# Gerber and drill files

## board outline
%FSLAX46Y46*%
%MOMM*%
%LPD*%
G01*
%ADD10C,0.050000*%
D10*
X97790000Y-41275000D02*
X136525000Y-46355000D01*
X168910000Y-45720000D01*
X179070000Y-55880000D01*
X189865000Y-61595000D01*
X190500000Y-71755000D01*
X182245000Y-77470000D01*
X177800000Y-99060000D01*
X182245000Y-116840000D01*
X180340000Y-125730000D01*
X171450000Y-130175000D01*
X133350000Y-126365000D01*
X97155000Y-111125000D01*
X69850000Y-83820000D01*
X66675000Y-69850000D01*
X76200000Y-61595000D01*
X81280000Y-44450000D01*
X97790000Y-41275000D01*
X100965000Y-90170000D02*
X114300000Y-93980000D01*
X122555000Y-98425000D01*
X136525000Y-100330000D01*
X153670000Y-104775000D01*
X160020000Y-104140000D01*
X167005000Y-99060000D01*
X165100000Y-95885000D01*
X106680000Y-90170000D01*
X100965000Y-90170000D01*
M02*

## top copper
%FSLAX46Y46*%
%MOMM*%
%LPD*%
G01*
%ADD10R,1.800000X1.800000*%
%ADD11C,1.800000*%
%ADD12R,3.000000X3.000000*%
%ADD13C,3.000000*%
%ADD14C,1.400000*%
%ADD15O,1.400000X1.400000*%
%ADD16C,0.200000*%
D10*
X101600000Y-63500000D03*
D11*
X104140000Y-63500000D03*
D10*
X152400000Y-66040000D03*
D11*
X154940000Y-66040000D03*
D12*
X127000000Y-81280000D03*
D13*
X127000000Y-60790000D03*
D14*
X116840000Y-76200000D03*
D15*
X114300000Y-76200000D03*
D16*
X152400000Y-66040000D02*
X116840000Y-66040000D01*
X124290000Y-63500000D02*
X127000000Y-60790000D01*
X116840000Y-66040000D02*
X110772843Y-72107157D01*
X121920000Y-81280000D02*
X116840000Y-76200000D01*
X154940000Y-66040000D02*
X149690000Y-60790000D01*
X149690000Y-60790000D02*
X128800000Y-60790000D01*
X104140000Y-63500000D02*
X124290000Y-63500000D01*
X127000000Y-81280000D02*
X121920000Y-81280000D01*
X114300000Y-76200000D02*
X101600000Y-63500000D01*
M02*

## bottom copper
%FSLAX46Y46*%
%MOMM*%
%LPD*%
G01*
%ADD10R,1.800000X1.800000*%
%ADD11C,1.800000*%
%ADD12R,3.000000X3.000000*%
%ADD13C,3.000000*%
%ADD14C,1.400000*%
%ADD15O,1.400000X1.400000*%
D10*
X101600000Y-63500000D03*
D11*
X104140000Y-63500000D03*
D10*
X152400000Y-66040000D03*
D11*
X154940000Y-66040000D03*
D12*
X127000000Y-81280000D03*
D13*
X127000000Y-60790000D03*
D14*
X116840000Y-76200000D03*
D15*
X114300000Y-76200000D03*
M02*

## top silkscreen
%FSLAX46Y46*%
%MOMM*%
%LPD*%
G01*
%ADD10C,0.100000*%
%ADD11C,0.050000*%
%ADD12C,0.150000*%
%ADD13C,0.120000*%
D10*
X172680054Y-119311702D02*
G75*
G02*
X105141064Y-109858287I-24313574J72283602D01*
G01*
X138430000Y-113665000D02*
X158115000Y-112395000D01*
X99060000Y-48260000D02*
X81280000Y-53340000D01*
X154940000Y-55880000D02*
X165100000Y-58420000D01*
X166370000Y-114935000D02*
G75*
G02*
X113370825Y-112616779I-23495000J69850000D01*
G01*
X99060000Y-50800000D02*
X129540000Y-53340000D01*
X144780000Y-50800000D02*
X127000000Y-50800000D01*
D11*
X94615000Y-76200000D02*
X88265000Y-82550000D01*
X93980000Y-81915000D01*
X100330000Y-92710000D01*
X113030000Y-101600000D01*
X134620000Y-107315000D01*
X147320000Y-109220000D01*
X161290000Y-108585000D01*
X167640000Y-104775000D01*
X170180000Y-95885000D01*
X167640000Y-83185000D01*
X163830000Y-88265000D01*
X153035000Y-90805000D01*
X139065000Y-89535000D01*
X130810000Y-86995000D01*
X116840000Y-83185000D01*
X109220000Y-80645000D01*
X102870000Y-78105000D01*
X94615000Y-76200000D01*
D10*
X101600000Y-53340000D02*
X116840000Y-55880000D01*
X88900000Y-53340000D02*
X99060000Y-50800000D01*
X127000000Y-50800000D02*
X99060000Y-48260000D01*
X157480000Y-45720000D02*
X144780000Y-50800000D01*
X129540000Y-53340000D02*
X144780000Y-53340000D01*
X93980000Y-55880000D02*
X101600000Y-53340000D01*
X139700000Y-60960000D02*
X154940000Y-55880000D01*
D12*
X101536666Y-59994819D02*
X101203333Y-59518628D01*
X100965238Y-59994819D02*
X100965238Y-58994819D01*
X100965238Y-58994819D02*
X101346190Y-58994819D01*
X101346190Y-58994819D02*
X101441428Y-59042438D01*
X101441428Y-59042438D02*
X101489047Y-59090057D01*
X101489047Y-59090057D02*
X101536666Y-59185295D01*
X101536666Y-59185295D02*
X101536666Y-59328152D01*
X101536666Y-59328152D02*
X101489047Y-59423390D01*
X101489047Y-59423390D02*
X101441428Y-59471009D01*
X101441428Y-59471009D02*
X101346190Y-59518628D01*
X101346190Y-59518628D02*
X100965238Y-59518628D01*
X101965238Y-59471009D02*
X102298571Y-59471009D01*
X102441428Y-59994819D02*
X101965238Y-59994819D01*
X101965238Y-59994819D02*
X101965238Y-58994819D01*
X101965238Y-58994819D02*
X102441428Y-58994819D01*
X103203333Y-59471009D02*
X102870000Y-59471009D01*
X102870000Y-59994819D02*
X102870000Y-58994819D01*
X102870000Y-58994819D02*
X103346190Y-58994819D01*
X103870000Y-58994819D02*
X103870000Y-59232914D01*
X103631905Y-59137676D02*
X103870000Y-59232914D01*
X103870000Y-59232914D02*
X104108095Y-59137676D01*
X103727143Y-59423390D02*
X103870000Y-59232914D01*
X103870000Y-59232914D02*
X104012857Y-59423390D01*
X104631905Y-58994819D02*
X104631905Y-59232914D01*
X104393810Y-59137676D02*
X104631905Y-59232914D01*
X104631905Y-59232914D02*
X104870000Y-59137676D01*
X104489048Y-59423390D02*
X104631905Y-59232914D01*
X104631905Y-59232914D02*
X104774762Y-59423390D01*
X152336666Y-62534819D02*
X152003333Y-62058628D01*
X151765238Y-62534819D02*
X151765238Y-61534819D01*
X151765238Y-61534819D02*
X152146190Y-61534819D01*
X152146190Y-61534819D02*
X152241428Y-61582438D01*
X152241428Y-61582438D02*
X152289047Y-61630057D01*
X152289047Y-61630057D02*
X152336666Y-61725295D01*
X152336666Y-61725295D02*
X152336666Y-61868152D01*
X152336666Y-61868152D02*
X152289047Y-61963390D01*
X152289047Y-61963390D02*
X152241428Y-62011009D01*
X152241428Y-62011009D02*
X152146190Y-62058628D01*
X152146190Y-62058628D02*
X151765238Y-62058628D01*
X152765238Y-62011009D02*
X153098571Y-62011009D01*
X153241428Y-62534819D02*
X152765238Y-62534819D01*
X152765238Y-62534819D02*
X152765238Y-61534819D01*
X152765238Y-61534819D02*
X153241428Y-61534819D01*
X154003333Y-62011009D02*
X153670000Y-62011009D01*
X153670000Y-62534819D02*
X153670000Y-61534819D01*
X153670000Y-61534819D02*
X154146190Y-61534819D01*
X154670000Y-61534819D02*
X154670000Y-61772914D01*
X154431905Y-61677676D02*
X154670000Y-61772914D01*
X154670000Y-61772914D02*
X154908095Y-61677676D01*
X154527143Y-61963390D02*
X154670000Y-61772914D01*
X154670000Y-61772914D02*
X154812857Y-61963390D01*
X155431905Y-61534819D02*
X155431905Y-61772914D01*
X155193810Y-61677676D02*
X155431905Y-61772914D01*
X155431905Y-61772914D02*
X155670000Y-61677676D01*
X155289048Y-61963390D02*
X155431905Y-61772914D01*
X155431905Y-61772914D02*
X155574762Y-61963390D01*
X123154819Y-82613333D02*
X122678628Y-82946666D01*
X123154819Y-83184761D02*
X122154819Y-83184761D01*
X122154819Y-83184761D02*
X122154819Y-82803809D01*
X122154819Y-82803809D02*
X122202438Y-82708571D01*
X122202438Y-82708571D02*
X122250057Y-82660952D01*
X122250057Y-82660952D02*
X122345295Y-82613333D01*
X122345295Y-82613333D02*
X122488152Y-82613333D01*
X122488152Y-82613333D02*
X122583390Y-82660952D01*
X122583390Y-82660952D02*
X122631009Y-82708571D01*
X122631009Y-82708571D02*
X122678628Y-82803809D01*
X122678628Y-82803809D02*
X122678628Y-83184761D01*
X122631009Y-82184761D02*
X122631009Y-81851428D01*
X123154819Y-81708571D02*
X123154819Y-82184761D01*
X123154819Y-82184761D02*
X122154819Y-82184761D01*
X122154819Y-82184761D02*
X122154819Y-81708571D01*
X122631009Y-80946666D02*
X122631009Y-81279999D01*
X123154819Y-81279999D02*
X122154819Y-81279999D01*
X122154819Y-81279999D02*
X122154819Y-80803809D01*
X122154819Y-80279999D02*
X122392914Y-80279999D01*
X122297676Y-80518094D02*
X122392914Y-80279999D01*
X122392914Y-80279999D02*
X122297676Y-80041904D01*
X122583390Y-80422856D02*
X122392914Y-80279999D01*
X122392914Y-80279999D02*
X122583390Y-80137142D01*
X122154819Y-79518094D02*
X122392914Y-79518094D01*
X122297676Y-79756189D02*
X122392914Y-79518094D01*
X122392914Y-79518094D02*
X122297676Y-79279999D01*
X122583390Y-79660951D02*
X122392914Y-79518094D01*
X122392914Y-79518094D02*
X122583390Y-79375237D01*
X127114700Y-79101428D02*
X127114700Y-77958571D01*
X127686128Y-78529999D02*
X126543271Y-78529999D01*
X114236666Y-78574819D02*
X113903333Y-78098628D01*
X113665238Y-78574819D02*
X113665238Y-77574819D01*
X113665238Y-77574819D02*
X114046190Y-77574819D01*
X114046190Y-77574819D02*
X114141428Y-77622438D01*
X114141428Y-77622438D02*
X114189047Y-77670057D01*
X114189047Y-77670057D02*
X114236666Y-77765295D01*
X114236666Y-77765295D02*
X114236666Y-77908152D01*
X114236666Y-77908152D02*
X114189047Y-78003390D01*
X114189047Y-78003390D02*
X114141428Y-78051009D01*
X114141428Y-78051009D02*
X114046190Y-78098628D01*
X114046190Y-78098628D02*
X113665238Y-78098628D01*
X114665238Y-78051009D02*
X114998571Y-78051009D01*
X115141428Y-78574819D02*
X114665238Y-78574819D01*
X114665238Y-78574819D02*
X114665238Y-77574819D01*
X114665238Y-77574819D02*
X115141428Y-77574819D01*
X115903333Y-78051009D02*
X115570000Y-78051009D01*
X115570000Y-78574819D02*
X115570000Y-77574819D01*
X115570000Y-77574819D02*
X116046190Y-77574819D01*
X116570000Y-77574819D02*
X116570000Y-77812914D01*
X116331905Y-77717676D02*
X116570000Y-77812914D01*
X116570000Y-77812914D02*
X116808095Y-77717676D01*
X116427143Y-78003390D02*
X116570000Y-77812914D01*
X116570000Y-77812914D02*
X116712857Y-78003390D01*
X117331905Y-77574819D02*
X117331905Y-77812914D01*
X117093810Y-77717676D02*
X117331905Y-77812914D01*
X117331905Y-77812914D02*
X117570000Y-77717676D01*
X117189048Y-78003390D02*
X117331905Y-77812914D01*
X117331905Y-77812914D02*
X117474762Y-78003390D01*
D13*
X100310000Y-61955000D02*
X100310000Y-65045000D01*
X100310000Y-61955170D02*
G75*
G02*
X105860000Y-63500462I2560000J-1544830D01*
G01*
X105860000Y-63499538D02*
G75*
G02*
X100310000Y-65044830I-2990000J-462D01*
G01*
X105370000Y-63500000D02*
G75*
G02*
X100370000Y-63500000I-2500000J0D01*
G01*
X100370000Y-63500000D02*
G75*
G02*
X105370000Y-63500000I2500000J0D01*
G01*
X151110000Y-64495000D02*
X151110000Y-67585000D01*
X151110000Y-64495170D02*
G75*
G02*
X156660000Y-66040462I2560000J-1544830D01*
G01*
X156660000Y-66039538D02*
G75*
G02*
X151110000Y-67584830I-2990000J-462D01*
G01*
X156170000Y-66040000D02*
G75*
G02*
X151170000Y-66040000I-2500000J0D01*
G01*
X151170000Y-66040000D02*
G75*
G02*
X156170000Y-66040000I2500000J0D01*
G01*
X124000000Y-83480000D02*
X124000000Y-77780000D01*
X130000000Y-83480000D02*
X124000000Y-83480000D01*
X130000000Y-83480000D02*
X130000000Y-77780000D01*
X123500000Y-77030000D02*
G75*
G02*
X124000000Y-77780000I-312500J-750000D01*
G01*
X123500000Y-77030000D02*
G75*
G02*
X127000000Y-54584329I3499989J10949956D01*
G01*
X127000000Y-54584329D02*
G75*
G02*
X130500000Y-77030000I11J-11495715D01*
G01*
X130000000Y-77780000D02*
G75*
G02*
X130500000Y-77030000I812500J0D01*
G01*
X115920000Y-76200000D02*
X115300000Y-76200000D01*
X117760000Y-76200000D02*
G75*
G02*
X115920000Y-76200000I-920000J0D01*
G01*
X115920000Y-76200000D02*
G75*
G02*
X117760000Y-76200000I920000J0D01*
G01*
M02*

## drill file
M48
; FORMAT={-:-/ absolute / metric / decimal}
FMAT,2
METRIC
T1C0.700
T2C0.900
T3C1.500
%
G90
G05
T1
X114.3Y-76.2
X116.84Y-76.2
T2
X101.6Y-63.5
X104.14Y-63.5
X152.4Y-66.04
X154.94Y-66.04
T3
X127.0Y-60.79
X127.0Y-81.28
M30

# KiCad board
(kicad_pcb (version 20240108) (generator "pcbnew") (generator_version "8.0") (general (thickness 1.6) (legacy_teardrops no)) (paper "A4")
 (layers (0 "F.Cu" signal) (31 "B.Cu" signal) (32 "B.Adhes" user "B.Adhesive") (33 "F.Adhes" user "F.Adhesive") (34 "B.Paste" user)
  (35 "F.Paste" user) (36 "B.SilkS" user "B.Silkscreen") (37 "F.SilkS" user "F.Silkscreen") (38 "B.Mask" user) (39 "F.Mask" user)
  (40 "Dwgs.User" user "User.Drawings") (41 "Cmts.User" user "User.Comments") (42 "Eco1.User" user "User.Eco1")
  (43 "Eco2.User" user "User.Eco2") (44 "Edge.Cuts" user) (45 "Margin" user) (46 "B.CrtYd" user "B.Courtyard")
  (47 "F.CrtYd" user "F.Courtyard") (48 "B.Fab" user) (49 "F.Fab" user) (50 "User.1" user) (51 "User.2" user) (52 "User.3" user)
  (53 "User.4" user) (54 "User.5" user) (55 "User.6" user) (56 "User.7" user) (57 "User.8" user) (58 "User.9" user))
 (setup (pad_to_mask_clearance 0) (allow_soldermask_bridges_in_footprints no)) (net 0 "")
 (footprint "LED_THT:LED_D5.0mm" (layer "F.Cu") (at 101.6 63.5)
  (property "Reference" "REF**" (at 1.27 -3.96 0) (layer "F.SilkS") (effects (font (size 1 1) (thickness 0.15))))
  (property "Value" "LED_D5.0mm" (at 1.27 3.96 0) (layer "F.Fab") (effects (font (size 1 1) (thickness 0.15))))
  (fp_line (start -1.29 -1.545) (end -1.29 1.545) (stroke (width 0.12) (type solid)) (layer "F.SilkS"))
  (fp_arc (start -1.29 -1.54483) (mid 2.072002 -2.880433) (end 4.26 0.000462) (stroke (width 0.12) (type solid)) (layer "F.SilkS"))
  (fp_arc (start 4.26 -0.000462) (mid 2.072002 2.880433) (end -1.29 1.54483) (stroke (width 0.12) (type solid)) (layer "F.SilkS"))
  (fp_circle (center 1.27 0) (end 3.77 0) (stroke (width 0.12) (type solid)) (fill none) (layer "F.SilkS"))
  (pad "1" thru_hole rect (at 0 0) (size 1.8 1.8) (drill 0.9) (layers "*.Cu" "*.Mask") (remove_unused_layers no))
  (pad "2" thru_hole circle (at 2.54 0) (size 1.8 1.8) (drill 0.9) (layers "*.Cu" "*.Mask") (remove_unused_layers no)))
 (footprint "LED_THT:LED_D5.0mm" (layer "F.Cu") (at 152.4 66.04)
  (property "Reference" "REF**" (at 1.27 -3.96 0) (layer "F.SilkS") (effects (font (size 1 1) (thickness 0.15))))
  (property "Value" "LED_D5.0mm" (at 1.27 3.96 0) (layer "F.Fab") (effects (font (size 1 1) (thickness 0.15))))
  (fp_line (start -1.29 -1.545) (end -1.29 1.545) (stroke (width 0.12) (type solid)) (layer "F.SilkS"))
  (fp_arc (start -1.29 -1.54483) (mid 2.072002 -2.880433) (end 4.26 0.000462) (stroke (width 0.12) (type solid)) (layer "F.SilkS"))
  (fp_arc (start 4.26 -0.000462) (mid 2.072002 2.880433) (end -1.29 1.54483) (stroke (width 0.12) (type solid)) (layer "F.SilkS"))
  (fp_circle (center 1.27 0) (end 3.77 0) (stroke (width 0.12) (type solid)) (fill none) (layer "F.SilkS"))
  (pad "1" thru_hole rect (at 0 0) (size 1.8 1.8) (drill 0.9) (layers "*.Cu" "*.Mask") (remove_unused_layers no))
  (pad "2" thru_hole circle (at 2.54 0) (size 1.8 1.8) (drill 0.9) (layers "*.Cu" "*.Mask") (remove_unused_layers no)))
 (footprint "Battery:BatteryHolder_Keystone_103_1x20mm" (layer "F.Cu") (at 127 81.28 90)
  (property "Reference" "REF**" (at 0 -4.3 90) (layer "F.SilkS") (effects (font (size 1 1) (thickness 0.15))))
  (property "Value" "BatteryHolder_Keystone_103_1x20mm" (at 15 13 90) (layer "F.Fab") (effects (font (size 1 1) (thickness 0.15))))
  (fp_line (start -2.2 -3) (end 3.5 -3) (stroke (width 0.12) (type solid)) (layer "F.SilkS"))
  (fp_line (start -2.2 3) (end -2.2 -3) (stroke (width 0.12) (type solid)) (layer "F.SilkS"))
  (fp_line (start -2.2 3) (end 3.5 3) (stroke (width 0.12) (type solid)) (layer "F.SilkS"))
  (fp_arc (start 4.25 -3.5) (mid 3.950694 -3.136459) (end 3.5 -3) (stroke (width 0.12) (type solid)) (layer "F.SilkS"))
  (fp_arc (start 4.25 -3.5) (mid 16.971103 -11.358466) (end 26.695671 0) (stroke (width 0.12) (type solid)) (layer "F.SilkS"))
  (fp_arc (start 26.695671 0) (mid 16.971103 11.358466) (end 4.25 3.5) (stroke (width 0.12) (type solid)) (layer "F.SilkS"))
  (fp_arc (start 3.5 3) (mid 3.950694 3.136459) (end 4.25 3.5) (stroke (width 0.12) (type solid)) (layer "F.SilkS"))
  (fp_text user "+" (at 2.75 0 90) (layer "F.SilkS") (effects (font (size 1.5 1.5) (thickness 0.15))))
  (pad "1" thru_hole rect (at 0 0 90) (size 3 3) (drill 1.5) (layers "*.Cu" "*.Mask") (remove_unused_layers no))
  (pad "2" thru_hole circle (at 20.49 0 90) (size 3 3) (drill 1.5) (layers "*.Cu" "*.Mask") (remove_unused_layers no)))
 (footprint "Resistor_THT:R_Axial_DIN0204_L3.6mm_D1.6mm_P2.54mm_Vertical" (layer "F.Cu") (at 116.84 76.2 180)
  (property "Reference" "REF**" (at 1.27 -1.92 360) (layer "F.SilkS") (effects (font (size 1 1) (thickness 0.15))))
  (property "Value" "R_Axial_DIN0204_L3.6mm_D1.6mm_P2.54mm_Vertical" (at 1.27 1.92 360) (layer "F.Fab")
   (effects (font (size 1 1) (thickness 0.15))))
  (fp_line (start 0.92 0) (end 1.54 0) (stroke (width 0.12) (type solid)) (layer "F.SilkS"))
  (fp_circle (center 0 0) (end 0.92 0) (stroke (width 0.12) (type solid)) (fill none) (layer "F.SilkS"))
  (pad "1" thru_hole circle (at 0 0 180) (size 1.4 1.4) (drill 0.7) (layers "*.Cu" "*.Mask") (remove_unused_layers no))
  (pad "2" thru_hole oval (at 2.54 0 180) (size 1.4 1.4) (drill 0.7) (layers "*.Cu" "*.Mask") (remove_unused_layers no)))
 (gr_arc (start 172.680054 119.311702) (mid 137.795 122.555) (end 105.141066 109.858285) (stroke (width 0.1) (type default))
  (layer "F.SilkS"))
 (gr_line (start 138.43 113.665) (end 158.115 112.395) (stroke (width 0.1) (type default)) (layer "F.SilkS"))
 (gr_line (start 99.06 48.26) (end 81.28 53.34) (stroke (width 0.1) (type default)) (layer "F.SilkS"))
 (gr_line (start 154.94 55.88) (end 165.1 58.42) (stroke (width 0.1) (type default)) (layer "F.SilkS"))
 (gr_arc (start 166.37 114.935) (mid 139.654583 118.710175) (end 113.370825 112.616779) (stroke (width 0.1) (type default))
  (layer "F.SilkS"))
 (gr_line (start 99.06 50.8) (end 129.54 53.34) (stroke (width 0.1) (type default)) (layer "F.SilkS"))
 (gr_line (start 144.78 50.8) (end 127 50.8) (stroke (width 0.1) (type default)) (layer "F.SilkS"))
 (gr_poly
  (pts (xy 94.615 76.2) (xy 88.265 82.55) (xy 93.98 81.915) (xy 100.33 92.71) (xy 113.03 101.6) (xy 134.62 107.315) (xy 147.32 109.22)
   (xy 161.29 108.585) (xy 167.64 104.775) (xy 170.18 95.885) (xy 167.64 83.185) (xy 163.83 88.265) (xy 153.035 90.805) (xy 139.065 89.535)
   (xy 130.81 86.995) (xy 116.84 83.185) (xy 109.22 80.645) (xy 102.87 78.105))
  (stroke (width 0.05) (type solid)) (fill none) (layer "F.SilkS"))
 (gr_line (start 101.6 53.34) (end 116.84 55.88) (stroke (width 0.1) (type default)) (layer "F.SilkS"))
 (gr_line (start 88.9 53.34) (end 99.06 50.8) (stroke (width 0.1) (type default)) (layer "F.SilkS"))
 (gr_line (start 127 50.8) (end 99.06 48.26) (stroke (width 0.1) (type default)) (layer "F.SilkS"))
 (gr_line (start 157.48 45.72) (end 144.78 50.8) (stroke (width 0.1) (type default)) (layer "F.SilkS"))
 (gr_line (start 129.54 53.34) (end 144.78 53.34) (stroke (width 0.1) (type default)) (layer "F.SilkS"))
 (gr_line (start 93.98 55.88) (end 101.6 53.34) (stroke (width 0.1) (type default)) (layer "F.SilkS"))
 (gr_line (start 139.7 60.96) (end 154.94 55.88) (stroke (width 0.1) (type default)) (layer "F.SilkS"))
 (gr_poly
  (pts (xy 97.79 41.275) (xy 136.525 46.355) (xy 168.91 45.72) (xy 179.07 55.88) (xy 189.865 61.595) (xy 190.5 71.755) (xy 182.245 77.47)
   (xy 177.8 99.06) (xy 182.245 116.84) (xy 180.34 125.73) (xy 171.45 130.175) (xy 133.35 126.365) (xy 97.155 111.125) (xy 69.85 83.82)
   (xy 66.675 69.85) (xy 76.2 61.595) (xy 81.28 44.45))
  (stroke (width 0.05) (type solid)) (fill none) (layer "Edge.Cuts"))
 (gr_poly
  (pts (xy 100.965 90.17) (xy 114.3 93.98) (xy 122.555 98.425) (xy 136.525 100.33) (xy 153.67 104.775) (xy 160.02 104.14) (xy 167.005 99.06)
   (xy 165.1 95.885) (xy 106.68 90.17))
  (stroke (width 0.05) (type solid)) (fill none) (layer "Edge.Cuts"))
 (segment (start 152.4 66.04) (end 116.84 66.04) (width 0.2) (layer "F.Cu") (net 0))
 (segment (start 124.29 63.5) (end 127 60.79) (width 0.2) (layer "F.Cu") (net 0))
 (segment (start 116.84 66.04) (end 110.772843 72.107157) (width 0.2) (layer "F.Cu") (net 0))
 (segment (start 121.92 81.28) (end 116.84 76.2) (width 0.2) (layer "F.Cu") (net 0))
 (segment (start 154.94 66.04) (end 149.69 60.79) (width 0.2) (layer "F.Cu") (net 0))
 (segment (start 149.69 60.79) (end 128.8 60.79) (width 0.2) (layer "F.Cu") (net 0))
 (segment (start 104.14 63.5) (end 124.29 63.5) (width 0.2) (layer "F.Cu") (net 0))
 (segment (start 127 81.28) (end 121.92 81.28) (width 0.2) (layer "F.Cu") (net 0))
 (segment (start 114.3 76.2) (end 101.6 63.5) (width 0.2) (layer "F.Cu") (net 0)))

